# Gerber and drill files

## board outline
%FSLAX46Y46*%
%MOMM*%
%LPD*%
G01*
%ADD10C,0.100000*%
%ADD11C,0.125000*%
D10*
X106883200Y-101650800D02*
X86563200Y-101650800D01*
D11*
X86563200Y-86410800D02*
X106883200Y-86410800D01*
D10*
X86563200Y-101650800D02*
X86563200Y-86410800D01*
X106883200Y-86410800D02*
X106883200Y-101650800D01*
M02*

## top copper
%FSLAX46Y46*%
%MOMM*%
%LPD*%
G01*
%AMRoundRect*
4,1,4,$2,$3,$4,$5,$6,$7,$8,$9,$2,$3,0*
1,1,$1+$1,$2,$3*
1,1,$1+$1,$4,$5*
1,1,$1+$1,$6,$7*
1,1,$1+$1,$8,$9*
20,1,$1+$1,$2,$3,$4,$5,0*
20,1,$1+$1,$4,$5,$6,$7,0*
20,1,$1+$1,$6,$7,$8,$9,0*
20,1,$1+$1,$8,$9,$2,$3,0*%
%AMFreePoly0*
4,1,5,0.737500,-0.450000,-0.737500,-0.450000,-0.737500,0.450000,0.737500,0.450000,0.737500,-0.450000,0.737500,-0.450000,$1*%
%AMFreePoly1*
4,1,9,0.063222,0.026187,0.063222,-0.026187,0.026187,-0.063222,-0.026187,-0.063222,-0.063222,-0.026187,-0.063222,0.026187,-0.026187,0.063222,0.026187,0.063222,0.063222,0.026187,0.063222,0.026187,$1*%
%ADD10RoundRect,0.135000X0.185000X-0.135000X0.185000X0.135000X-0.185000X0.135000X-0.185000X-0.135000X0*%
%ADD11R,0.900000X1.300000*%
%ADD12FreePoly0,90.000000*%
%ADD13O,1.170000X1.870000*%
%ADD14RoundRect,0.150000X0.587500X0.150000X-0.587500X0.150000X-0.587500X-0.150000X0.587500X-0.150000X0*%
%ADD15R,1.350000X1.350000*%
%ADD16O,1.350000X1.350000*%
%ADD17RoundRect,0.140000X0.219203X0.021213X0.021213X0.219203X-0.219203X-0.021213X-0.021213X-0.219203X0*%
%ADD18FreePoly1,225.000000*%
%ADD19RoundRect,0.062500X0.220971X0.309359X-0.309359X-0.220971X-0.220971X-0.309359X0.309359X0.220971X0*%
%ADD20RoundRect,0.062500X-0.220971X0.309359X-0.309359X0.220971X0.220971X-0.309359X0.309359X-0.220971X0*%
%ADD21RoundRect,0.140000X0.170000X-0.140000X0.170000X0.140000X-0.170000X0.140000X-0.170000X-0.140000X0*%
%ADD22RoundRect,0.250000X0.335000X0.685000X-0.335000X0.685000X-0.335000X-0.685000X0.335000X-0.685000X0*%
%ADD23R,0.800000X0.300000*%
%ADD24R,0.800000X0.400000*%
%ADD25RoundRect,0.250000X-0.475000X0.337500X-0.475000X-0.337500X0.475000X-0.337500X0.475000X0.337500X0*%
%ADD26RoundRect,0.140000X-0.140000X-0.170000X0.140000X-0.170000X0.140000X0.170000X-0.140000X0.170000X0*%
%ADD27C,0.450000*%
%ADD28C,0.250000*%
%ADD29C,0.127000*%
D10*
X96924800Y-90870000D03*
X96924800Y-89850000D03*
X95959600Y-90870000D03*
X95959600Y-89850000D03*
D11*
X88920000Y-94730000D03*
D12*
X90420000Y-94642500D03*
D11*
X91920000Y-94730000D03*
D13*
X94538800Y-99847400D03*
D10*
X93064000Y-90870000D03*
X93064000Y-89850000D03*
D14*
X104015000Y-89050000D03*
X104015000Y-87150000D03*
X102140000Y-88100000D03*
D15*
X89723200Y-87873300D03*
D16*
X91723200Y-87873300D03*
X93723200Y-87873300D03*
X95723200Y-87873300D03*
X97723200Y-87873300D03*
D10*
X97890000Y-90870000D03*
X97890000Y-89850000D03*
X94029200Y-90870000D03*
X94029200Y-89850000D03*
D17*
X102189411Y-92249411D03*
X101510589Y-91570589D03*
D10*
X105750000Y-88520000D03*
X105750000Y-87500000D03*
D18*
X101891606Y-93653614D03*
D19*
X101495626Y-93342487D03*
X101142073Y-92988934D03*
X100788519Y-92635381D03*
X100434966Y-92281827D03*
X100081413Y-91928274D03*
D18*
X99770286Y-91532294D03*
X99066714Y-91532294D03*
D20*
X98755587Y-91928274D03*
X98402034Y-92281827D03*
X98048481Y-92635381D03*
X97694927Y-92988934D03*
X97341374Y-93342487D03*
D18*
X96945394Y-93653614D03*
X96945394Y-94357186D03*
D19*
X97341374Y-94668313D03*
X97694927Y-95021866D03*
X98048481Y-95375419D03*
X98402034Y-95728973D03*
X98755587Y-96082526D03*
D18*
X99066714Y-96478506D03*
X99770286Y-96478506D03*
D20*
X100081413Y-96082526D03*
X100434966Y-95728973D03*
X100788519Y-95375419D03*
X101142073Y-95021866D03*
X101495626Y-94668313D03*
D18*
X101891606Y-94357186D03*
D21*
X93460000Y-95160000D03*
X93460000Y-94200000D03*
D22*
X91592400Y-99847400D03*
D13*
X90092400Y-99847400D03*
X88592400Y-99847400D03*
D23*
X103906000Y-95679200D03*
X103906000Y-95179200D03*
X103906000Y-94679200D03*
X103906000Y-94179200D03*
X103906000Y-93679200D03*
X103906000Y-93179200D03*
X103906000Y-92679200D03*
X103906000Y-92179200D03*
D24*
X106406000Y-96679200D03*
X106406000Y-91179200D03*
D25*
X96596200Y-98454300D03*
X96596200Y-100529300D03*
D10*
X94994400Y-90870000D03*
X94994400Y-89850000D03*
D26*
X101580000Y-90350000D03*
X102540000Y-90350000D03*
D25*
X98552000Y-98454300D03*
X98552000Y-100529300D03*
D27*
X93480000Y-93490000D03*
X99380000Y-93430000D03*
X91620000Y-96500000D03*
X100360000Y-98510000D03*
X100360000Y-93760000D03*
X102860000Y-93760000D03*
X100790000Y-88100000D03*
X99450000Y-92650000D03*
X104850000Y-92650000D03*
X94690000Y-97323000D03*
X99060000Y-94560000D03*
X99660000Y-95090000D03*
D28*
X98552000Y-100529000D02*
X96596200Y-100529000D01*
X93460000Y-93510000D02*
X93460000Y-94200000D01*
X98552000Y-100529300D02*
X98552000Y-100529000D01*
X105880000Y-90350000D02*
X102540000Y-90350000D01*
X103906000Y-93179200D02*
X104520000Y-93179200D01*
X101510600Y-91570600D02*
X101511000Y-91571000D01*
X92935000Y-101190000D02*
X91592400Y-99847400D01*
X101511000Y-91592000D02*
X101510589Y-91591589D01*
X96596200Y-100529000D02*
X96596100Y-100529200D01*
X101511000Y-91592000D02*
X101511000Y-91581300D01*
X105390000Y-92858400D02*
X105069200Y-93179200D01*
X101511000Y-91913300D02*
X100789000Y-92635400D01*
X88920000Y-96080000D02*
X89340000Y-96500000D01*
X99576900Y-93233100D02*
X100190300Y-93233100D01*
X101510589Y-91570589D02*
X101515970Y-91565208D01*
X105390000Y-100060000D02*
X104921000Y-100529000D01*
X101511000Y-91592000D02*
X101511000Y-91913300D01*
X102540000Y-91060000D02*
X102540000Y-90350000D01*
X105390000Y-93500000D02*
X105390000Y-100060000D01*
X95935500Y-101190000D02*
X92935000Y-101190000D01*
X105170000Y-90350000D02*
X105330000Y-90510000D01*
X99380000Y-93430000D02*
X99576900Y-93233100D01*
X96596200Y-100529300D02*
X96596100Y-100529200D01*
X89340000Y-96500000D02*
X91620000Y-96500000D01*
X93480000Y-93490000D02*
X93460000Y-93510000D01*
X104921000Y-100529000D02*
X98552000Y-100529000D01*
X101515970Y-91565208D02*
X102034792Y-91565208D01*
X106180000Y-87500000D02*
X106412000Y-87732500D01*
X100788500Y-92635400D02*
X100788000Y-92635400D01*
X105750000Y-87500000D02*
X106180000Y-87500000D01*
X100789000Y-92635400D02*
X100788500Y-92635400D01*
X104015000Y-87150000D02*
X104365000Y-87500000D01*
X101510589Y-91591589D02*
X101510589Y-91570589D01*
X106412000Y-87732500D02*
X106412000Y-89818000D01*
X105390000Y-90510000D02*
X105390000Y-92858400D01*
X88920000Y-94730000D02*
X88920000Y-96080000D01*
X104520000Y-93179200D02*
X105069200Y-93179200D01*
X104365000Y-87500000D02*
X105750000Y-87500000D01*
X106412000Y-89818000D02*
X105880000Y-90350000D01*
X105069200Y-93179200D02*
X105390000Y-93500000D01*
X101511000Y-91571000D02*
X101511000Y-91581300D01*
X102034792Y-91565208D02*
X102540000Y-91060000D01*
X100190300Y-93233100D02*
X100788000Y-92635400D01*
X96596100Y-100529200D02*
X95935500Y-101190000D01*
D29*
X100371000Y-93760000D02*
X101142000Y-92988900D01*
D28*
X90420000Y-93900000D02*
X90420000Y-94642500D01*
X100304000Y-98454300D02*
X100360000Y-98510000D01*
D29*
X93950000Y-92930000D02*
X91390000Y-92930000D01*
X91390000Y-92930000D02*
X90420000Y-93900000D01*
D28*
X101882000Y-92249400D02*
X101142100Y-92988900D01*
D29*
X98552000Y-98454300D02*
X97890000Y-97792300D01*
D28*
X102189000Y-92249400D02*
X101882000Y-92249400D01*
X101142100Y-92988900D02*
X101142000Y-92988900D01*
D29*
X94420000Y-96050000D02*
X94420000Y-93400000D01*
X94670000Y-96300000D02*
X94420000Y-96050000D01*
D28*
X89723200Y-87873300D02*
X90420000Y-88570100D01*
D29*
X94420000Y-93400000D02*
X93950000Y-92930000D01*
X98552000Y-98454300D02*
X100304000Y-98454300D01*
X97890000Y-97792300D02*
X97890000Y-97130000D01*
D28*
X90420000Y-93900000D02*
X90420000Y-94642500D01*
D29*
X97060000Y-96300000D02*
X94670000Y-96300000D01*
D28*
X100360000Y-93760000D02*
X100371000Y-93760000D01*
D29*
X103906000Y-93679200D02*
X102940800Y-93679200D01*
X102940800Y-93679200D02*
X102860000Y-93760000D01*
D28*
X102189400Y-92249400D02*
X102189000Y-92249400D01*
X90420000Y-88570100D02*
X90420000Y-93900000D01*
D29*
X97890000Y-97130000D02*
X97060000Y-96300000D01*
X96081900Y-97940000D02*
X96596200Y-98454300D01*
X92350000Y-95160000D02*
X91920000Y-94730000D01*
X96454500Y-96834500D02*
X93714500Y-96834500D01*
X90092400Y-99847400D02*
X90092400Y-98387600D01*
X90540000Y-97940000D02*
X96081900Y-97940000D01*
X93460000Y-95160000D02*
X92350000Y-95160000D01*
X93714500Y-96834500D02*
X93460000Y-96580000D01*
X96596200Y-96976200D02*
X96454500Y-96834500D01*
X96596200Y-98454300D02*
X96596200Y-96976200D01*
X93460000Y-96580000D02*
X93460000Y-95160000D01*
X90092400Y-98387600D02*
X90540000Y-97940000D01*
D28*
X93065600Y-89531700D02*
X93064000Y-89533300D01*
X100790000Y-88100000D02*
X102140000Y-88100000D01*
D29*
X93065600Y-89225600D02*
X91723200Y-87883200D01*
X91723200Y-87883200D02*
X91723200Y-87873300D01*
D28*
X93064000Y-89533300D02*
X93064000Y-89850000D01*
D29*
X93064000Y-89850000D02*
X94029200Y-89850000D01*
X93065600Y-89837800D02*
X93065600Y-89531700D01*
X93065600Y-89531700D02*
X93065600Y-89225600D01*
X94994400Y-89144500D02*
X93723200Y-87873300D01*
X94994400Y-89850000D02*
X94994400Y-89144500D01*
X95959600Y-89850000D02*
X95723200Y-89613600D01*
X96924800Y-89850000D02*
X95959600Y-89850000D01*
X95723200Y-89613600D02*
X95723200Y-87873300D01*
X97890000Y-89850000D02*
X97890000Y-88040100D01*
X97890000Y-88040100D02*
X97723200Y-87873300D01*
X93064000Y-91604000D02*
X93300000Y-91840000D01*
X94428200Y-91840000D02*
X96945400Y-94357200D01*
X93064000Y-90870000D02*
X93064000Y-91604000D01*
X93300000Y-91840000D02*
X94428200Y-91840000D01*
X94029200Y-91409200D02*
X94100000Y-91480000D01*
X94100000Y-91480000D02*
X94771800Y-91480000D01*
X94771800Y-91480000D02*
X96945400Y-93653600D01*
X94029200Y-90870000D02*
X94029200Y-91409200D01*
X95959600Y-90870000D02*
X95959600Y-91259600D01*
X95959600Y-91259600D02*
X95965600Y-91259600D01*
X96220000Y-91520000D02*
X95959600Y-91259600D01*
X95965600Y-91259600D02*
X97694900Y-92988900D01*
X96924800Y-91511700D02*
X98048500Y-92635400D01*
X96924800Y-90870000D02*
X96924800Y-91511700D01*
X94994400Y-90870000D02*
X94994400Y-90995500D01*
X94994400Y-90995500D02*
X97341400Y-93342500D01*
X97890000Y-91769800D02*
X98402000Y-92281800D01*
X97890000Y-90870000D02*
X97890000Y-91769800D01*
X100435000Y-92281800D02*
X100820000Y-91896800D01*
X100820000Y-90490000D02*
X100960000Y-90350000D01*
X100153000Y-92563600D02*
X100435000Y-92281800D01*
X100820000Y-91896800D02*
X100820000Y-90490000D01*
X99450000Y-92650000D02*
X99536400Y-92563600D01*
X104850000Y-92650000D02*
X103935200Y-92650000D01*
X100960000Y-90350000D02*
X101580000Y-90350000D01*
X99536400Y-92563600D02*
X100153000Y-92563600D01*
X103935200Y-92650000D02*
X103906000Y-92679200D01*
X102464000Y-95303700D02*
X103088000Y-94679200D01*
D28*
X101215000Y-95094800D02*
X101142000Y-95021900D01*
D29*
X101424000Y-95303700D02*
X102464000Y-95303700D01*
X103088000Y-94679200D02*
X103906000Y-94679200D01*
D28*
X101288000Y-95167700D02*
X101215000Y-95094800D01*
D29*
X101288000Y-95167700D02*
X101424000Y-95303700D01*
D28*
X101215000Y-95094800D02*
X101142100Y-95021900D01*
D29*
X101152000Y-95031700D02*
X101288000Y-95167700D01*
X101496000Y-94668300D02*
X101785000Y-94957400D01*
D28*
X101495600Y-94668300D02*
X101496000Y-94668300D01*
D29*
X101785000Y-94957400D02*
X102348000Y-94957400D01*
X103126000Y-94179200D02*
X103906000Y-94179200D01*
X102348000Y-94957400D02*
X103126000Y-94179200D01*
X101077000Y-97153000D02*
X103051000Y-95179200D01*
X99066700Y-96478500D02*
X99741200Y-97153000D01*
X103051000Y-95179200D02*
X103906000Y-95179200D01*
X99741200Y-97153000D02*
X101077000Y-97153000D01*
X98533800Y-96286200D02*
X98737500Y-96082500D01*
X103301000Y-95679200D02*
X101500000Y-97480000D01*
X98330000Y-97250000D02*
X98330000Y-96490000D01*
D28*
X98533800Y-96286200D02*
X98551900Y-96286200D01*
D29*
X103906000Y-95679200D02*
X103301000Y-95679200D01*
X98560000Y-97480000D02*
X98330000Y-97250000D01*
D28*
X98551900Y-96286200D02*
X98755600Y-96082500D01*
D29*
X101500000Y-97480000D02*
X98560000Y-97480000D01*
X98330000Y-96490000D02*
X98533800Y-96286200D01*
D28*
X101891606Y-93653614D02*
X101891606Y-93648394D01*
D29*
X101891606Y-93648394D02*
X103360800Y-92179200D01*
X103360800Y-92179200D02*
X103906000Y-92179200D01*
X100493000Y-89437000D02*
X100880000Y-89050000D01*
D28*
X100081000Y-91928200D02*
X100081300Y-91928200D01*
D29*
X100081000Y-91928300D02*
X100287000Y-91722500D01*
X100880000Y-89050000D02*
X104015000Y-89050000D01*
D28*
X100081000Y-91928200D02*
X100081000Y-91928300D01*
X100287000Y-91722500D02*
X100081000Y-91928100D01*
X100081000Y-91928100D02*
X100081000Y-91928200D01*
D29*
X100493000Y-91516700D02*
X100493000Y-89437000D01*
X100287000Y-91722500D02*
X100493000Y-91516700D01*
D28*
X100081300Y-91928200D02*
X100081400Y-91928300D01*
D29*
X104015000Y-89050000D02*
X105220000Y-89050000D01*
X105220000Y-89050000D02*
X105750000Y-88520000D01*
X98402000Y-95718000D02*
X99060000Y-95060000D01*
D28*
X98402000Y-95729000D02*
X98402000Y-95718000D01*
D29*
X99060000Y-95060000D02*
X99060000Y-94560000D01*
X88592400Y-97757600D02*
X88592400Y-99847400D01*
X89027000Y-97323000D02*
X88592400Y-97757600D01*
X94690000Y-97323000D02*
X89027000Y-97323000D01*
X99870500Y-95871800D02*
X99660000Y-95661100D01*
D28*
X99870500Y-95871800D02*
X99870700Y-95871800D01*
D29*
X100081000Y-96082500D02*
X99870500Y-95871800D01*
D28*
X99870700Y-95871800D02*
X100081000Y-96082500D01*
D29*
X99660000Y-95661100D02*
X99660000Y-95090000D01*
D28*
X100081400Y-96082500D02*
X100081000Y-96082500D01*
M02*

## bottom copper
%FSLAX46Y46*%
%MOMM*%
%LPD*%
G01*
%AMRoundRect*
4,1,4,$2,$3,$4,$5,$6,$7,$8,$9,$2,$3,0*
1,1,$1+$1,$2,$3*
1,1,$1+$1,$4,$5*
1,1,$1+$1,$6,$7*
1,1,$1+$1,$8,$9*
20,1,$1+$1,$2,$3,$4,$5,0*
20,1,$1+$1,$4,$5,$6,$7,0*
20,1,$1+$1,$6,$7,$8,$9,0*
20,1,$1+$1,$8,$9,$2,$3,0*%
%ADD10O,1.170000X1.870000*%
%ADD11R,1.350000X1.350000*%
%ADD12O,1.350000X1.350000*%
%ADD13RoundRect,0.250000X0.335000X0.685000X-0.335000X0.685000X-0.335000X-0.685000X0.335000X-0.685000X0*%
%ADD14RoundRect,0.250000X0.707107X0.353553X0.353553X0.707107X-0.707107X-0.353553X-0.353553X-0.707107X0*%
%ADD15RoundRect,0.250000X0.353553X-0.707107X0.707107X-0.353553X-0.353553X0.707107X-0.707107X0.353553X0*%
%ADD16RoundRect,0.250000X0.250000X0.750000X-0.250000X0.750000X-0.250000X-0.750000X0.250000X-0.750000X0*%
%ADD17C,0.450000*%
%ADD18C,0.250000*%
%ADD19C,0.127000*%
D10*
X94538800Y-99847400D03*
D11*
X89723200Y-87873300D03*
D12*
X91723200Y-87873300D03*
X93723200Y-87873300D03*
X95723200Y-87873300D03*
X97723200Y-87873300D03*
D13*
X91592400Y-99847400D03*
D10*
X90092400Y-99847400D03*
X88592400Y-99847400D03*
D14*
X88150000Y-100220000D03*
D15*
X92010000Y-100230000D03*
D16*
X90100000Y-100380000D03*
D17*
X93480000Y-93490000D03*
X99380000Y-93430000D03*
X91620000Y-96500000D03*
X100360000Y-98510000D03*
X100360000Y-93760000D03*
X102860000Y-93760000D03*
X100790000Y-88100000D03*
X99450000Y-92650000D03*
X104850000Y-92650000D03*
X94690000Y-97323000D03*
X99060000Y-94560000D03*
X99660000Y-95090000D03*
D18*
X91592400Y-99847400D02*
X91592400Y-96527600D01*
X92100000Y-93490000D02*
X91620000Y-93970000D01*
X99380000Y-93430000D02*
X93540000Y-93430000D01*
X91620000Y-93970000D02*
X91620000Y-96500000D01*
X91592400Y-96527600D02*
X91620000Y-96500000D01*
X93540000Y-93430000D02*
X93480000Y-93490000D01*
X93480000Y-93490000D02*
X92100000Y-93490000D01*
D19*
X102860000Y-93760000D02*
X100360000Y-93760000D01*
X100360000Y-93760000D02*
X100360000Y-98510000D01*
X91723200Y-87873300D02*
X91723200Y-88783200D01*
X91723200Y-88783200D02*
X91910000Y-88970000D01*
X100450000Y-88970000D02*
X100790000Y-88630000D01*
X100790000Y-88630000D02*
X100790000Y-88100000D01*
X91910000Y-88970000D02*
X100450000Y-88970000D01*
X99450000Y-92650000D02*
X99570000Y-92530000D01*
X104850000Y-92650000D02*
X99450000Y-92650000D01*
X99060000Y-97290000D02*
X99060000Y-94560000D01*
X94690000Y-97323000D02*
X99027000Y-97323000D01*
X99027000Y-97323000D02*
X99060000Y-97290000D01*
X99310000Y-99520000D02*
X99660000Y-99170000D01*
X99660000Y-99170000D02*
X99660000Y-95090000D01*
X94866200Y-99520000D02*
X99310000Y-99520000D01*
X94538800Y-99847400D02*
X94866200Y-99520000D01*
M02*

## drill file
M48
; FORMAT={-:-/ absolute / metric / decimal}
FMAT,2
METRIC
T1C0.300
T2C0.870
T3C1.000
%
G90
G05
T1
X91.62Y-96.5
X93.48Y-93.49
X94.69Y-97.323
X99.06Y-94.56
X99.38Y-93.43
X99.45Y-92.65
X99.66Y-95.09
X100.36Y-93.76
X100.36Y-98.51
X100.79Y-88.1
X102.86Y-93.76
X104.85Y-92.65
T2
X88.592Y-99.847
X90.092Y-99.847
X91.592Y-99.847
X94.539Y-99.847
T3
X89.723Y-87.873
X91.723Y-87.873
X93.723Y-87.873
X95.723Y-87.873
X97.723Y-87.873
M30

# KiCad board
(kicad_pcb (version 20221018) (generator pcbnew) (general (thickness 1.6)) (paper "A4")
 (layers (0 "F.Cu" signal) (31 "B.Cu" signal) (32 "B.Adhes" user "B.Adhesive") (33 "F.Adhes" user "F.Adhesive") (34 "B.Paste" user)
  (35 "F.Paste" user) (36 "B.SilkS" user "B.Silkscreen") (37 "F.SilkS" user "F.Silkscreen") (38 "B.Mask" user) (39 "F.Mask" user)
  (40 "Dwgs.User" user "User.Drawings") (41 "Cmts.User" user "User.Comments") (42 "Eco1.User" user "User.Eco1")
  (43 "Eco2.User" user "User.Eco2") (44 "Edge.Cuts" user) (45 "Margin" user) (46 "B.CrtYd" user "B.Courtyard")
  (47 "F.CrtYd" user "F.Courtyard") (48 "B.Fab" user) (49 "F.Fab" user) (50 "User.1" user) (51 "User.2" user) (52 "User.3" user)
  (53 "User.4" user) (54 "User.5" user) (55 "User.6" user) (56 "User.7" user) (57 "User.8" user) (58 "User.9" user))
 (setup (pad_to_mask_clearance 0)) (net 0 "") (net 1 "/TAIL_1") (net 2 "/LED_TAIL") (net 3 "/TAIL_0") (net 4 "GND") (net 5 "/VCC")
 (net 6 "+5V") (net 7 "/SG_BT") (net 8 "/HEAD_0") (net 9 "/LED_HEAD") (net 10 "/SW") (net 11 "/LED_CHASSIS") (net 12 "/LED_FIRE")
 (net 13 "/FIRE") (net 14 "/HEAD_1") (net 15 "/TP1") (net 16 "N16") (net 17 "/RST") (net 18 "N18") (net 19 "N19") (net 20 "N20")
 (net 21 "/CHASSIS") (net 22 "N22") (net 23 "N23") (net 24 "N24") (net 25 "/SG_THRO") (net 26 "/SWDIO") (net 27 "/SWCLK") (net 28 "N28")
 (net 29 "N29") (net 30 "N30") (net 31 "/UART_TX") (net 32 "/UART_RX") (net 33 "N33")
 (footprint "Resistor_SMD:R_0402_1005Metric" (layer "F.Cu") (at 96.9248 90.36 90)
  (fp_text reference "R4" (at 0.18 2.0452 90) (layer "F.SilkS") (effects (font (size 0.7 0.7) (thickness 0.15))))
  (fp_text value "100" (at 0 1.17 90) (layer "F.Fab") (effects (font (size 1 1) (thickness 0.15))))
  (pad "1" smd roundrect (at -0.51 0 90) (size 0.54 0.64) (layers "F.Cu" "F.Paste" "F.Mask") (roundrect_rratio 0.25) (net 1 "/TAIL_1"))
  (pad "2" smd roundrect (at 0.51 0 90) (size 0.54 0.64) (layers "F.Cu" "F.Paste" "F.Mask") (roundrect_rratio 0.25) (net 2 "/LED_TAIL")))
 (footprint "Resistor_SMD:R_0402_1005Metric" (layer "F.Cu") (at 95.9596 90.36 90)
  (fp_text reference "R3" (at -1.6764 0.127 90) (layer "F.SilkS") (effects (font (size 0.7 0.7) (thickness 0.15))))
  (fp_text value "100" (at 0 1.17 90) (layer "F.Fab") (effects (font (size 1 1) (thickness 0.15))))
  (pad "1" smd roundrect (at -0.51 0 90) (size 0.54 0.64) (layers "F.Cu" "F.Paste" "F.Mask") (roundrect_rratio 0.25) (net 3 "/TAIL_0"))
  (pad "2" smd roundrect (at 0.51 0 90) (size 0.54 0.64) (layers "F.Cu" "F.Paste" "F.Mask") (roundrect_rratio 0.25) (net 2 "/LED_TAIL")))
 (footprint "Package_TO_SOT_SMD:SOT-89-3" (layer "F.Cu") (at 90.42 92.78 90)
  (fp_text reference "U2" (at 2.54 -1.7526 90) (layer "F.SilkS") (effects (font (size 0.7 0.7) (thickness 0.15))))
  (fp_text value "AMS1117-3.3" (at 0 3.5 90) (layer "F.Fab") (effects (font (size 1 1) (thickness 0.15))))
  (pad "1" smd rect (at -1.95 -1.5 90) (size 1.3 0.9) (layers "F.Cu" "F.Paste" "F.Mask") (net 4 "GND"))
  (pad "2" smd custom (at -1.8625 0 90) (size 1.475 0.9) (layers "F.Cu" "F.Paste" "F.Mask") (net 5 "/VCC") (zone_connect 2)
   (thermal_bridge_angle 45) (options (clearance outline) (anchor rect)) (primitives))
  (pad "3" smd rect (at -1.95 1.5 90) (size 1.3 0.9) (layers "F.Cu" "F.Paste" "F.Mask") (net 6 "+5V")))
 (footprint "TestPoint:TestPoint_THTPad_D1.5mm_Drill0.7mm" (layer "F.Cu") (at 94.5388 99.8474)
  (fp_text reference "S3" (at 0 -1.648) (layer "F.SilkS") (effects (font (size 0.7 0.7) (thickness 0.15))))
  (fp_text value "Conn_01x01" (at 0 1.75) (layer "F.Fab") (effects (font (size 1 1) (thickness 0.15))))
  (pad "1" thru_hole oval (at 0 0) (size 1.17 1.87) (drill 0.87) (layers "*.Cu" "*.Mask") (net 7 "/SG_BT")))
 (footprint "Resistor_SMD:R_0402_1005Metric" (layer "F.Cu") (at 93.064 90.36 90)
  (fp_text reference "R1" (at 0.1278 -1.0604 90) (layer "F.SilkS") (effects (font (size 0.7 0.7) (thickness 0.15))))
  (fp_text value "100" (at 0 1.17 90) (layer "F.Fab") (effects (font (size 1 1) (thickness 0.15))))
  (pad "1" smd roundrect (at -0.51 0 90) (size 0.54 0.64) (layers "F.Cu" "F.Paste" "F.Mask") (roundrect_rratio 0.25) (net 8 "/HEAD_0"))
  (pad "2" smd roundrect (at 0.51 0 90) (size 0.54 0.64) (layers "F.Cu" "F.Paste" "F.Mask") (roundrect_rratio 0.25) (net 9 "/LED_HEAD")))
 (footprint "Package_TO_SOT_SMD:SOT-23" (layer "F.Cu") (at 103.0775 88.1 180)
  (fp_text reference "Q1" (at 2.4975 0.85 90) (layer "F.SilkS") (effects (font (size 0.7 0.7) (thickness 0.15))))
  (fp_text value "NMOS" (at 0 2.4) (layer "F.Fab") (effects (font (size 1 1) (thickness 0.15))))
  (pad "1" smd roundrect (at -0.9375 -0.95 180) (size 1.475 0.6) (layers "F.Cu" "F.Paste" "F.Mask") (roundrect_rratio 0.25) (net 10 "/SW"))
  (pad "2" smd roundrect (at -0.9375 0.95 180) (size 1.475 0.6) (layers "F.Cu" "F.Paste" "F.Mask") (roundrect_rratio 0.25) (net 4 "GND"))
  (pad "3" smd roundrect (at 0.9375 0 180) (size 1.475 0.6) (layers "F.Cu" "F.Paste" "F.Mask") (roundrect_rratio 0.25) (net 9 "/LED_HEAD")))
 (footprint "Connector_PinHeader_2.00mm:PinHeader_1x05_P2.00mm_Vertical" (layer "F.Cu") (at 89.7232 87.8733 90)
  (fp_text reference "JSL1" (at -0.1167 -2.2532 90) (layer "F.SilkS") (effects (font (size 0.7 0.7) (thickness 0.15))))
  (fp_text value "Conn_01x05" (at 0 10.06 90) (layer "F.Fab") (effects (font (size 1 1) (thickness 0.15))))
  (pad "1" thru_hole rect (at 0 0 90) (size 1.35 1.35) (drill 1) (layers "*.Cu" "*.Mask") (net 5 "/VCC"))
  (pad "2" thru_hole oval (at 0 2 90) (size 1.35 1.35) (drill 1) (layers "*.Cu" "*.Mask") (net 9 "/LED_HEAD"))
  (pad "3" thru_hole oval (at 0 4 90) (size 1.35 1.35) (drill 1) (layers "*.Cu" "*.Mask") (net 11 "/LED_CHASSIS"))
  (pad "4" thru_hole oval (at 0 6 90) (size 1.35 1.35) (drill 1) (layers "*.Cu" "*.Mask") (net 2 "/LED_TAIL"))
  (pad "5" thru_hole oval (at 0 8 90) (size 1.35 1.35) (drill 1) (layers "*.Cu" "*.Mask") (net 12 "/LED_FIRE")))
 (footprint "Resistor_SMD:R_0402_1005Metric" (layer "F.Cu") (at 97.89 90.36 90)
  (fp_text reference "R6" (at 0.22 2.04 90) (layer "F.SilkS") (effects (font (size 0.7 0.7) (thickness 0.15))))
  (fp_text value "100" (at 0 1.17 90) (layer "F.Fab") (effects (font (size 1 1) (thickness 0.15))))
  (pad "1" smd roundrect (at -0.51 0 90) (size 0.54 0.64) (layers "F.Cu" "F.Paste" "F.Mask") (roundrect_rratio 0.25) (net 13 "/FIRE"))
  (pad "2" smd roundrect (at 0.51 0 90) (size 0.54 0.64) (layers "F.Cu" "F.Paste" "F.Mask") (roundrect_rratio 0.25) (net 12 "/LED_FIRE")))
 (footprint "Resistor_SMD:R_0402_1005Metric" (layer "F.Cu") (at 94.0292 90.36 90)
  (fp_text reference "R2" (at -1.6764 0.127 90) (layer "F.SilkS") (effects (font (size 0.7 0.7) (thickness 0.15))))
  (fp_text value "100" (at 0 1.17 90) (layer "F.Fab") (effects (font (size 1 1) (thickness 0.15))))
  (pad "1" smd roundrect (at -0.51 0 90) (size 0.54 0.64) (layers "F.Cu" "F.Paste" "F.Mask") (roundrect_rratio 0.25) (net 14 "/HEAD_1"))
  (pad "2" smd roundrect (at 0.51 0 90) (size 0.54 0.64) (layers "F.Cu" "F.Paste" "F.Mask") (roundrect_rratio 0.25) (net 9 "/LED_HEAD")))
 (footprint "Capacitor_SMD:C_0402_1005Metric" (layer "F.Cu") (at 101.85 91.91 135)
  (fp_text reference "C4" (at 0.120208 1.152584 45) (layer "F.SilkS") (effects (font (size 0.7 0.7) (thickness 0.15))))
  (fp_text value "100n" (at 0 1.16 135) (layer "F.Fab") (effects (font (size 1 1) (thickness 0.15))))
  (pad "1" smd roundrect (at -0.48 0 135) (size 0.56 0.62) (layers "F.Cu" "F.Paste" "F.Mask") (roundrect_rratio 0.25) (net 5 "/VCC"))
  (pad "2" smd roundrect (at 0.48 0 135) (size 0.56 0.62) (layers "F.Cu" "F.Paste" "F.Mask") (roundrect_rratio 0.25) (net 4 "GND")))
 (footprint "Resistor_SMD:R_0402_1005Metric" (layer "F.Cu") (at 105.75 88.01 90)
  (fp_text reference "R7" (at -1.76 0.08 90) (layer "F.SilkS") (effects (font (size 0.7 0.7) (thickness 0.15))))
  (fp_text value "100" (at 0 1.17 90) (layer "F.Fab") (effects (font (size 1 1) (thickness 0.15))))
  (pad "1" smd roundrect (at -0.51 0 90) (size 0.54 0.64) (layers "F.Cu" "F.Paste" "F.Mask") (roundrect_rratio 0.25) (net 10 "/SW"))
  (pad "2" smd roundrect (at 0.51 0 90) (size 0.54 0.64) (layers "F.Cu" "F.Paste" "F.Mask") (roundrect_rratio 0.25) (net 4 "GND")))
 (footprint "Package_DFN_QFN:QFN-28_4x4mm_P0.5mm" (layer "F.Cu") (at 99.4185 94.0054 -135)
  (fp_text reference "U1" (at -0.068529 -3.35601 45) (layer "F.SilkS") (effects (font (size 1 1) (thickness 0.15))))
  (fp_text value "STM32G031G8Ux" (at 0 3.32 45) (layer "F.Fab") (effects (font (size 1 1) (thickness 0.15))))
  (pad "1" smd custom (at -1.9975 -1.5 225) (size 0.136863 0.136863) (layers "F.Cu" "F.Paste" "F.Mask") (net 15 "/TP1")
   (thermal_bridge_angle 45) (options (clearance outline) (anchor circle)) (primitives))
  (pad "2" smd roundrect (at -1.9375 -1 225) (size 0.875 0.25) (layers "F.Cu" "F.Paste" "F.Mask") (roundrect_rratio 0.25) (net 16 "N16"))
  (pad "3" smd roundrect (at -1.9375 -0.5 225) (size 0.875 0.25) (layers "F.Cu" "F.Paste" "F.Mask") (roundrect_rratio 0.25) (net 5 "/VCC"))
  (pad "4" smd roundrect (at -1.9375 0 225) (size 0.875 0.25) (layers "F.Cu" "F.Paste" "F.Mask") (roundrect_rratio 0.25) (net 4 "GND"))
  (pad "5" smd roundrect (at -1.9375 0.5 225) (size 0.875 0.25) (layers "F.Cu" "F.Paste" "F.Mask") (roundrect_rratio 0.25) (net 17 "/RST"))
  (pad "6" smd roundrect (at -1.9375 1 225) (size 0.875 0.25) (layers "F.Cu" "F.Paste" "F.Mask") (roundrect_rratio 0.25) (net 10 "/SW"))
  (pad "7" smd custom (at -1.9975 1.5 225) (size 0.136863 0.136863) (layers "F.Cu" "F.Paste" "F.Mask") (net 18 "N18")
   (thermal_bridge_angle 45) (options (clearance outline) (anchor circle)) (primitives))
  (pad "8" smd custom (at -1.5 1.9975 225) (size 0.136863 0.136863) (layers "F.Cu" "F.Paste" "F.Mask") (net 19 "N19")
   (thermal_bridge_angle 45) (options (clearance outline) (anchor circle)) (primitives))
  (pad "9" smd roundrect (at -1 1.9375 225) (size 0.25 0.875) (layers "F.Cu" "F.Paste" "F.Mask") (roundrect_rratio 0.25) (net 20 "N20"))
  (pad "10" smd roundrect (at -0.5 1.9375 225) (size 0.25 0.875) (layers "F.Cu" "F.Paste" "F.Mask") (roundrect_rratio 0.25) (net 13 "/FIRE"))
  (pad "11" smd roundrect (at 0 1.9375 225) (size 0.25 0.875) (layers "F.Cu" "F.Paste" "F.Mask") (roundrect_rratio 0.25) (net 1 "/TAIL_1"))
  (pad "12" smd roundrect (at 0.5 1.9375 225) (size 0.25 0.875) (layers "F.Cu" "F.Paste" "F.Mask") (roundrect_rratio 0.25) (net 3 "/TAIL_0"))
  (pad "13" smd roundrect (at 1 1.9375 225) (size 0.25 0.875) (layers "F.Cu" "F.Paste" "F.Mask") (roundrect_rratio 0.25) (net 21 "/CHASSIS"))
  (pad "14" smd custom (at 1.5 1.9975 225) (size 0.136863 0.136863) (layers "F.Cu" "F.Paste" "F.Mask") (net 14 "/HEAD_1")
   (thermal_bridge_angle 45) (options (clearance outline) (anchor circle)) (primitives))
  (pad "15" smd custom (at 1.9975 1.5 225) (size 0.136863 0.136863) (layers "F.Cu" "F.Paste" "F.Mask") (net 8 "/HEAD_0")
   (thermal_bridge_angle 45) (options (clearance outline) (anchor circle)) (primitives))
  (pad "16" smd roundrect (at 1.9375 1 225) (size 0.875 0.25) (layers "F.Cu" "F.Paste" "F.Mask") (roundrect_rratio 0.25) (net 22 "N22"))
  (pad "17" smd roundrect (at 1.9375 0.5 225) (size 0.875 0.25) (layers "F.Cu" "F.Paste" "F.Mask") (roundrect_rratio 0.25) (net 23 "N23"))
  (pad "18" smd roundrect (at 1.9375 0 225) (size 0.875 0.25) (layers "F.Cu" "F.Paste" "F.Mask") (roundrect_rratio 0.25) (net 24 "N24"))
  (pad "19" smd roundrect (at 1.9375 -0.5 225) (size 0.875 0.25) (layers "F.Cu" "F.Paste" "F.Mask") (roundrect_rratio 0.25)
   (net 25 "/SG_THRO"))
  (pad "20" smd roundrect (at 1.9375 -1 225) (size 0.875 0.25) (layers "F.Cu" "F.Paste" "F.Mask") (roundrect_rratio 0.25) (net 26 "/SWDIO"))
  (pad "21" smd custom (at 1.9975 -1.5 225) (size 0.136863 0.136863) (layers "F.Cu" "F.Paste" "F.Mask") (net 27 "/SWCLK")
   (thermal_bridge_angle 45) (options (clearance outline) (anchor circle)) (primitives))
  (pad "22" smd custom (at 1.5 -1.9975 225) (size 0.136863 0.136863) (layers "F.Cu" "F.Paste" "F.Mask") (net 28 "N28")
   (thermal_bridge_angle 45) (options (clearance outline) (anchor circle)) (primitives))
  (pad "23" smd roundrect (at 1 -1.9375 225) (size 0.25 0.875) (layers "F.Cu" "F.Paste" "F.Mask") (roundrect_rratio 0.25) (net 7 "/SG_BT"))
  (pad "24" smd roundrect (at 0.5 -1.9375 225) (size 0.25 0.875) (layers "F.Cu" "F.Paste" "F.Mask") (roundrect_rratio 0.25) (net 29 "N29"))
  (pad "25" smd roundrect (at 0 -1.9375 225) (size 0.25 0.875) (layers "F.Cu" "F.Paste" "F.Mask") (roundrect_rratio 0.25) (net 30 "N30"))
  (pad "26" smd roundrect (at -0.5 -1.9375 225) (size 0.25 0.875) (layers "F.Cu" "F.Paste" "F.Mask") (roundrect_rratio 0.25)
   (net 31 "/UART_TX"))
  (pad "27" smd roundrect (at -1 -1.9375 225) (size 0.25 0.875) (layers "F.Cu" "F.Paste" "F.Mask") (roundrect_rratio 0.25)
   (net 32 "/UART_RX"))
  (pad "28" smd custom (at -1.5 -1.9975 225) (size 0.136863 0.136863) (layers "F.Cu" "F.Paste" "F.Mask") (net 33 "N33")
   (thermal_bridge_angle 45) (options (clearance outline) (anchor circle)) (primitives)))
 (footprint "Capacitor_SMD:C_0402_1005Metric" (layer "F.Cu") (at 93.46 94.68 90)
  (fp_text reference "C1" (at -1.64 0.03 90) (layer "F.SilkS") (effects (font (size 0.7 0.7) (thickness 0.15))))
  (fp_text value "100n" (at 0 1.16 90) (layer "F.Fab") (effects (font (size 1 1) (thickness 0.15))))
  (pad "1" smd roundrect (at -0.48 0 90) (size 0.56 0.62) (layers "F.Cu" "F.Paste" "F.Mask") (roundrect_rratio 0.25) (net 6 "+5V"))
  (pad "2" smd roundrect (at 0.48 0 90) (size 0.56 0.62) (layers "F.Cu" "F.Paste" "F.Mask") (roundrect_rratio 0.25) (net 4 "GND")))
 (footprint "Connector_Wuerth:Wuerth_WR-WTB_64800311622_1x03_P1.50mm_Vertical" (layer "F.Cu") (at 91.5924 99.8474 180)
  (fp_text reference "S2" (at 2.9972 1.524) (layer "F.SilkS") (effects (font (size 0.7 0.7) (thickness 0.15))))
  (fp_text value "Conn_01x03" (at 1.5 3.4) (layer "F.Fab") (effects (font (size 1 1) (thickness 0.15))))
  (pad "1" thru_hole roundrect (at 0 0 180) (size 1.17 1.87) (drill 0.87) (layers "*.Cu" "*.Mask") (roundrect_rratio 0.213675) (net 4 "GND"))
  (pad "2" thru_hole oval (at 1.5 0 180) (size 1.17 1.87) (drill 0.87) (layers "*.Cu" "*.Mask") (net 6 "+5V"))
  (pad "3" thru_hole oval (at 3 0 180) (size 1.17 1.87) (drill 0.87) (layers "*.Cu" "*.Mask") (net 25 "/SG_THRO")))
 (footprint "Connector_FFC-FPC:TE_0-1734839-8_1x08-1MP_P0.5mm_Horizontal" (layer "F.Cu") (at 104.831 93.9292 90)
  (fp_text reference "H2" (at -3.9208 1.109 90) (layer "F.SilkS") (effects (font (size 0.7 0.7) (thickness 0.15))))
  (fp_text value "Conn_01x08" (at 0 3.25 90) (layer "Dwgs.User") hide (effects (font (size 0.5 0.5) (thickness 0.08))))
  (pad "1" smd rect (at -1.75 -0.925 90) (size 0.3 0.8) (layers "F.Cu" "F.Paste" "F.Mask") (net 26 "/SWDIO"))
  (pad "2" smd rect (at -1.25 -0.925 90) (size 0.3 0.8) (layers "F.Cu" "F.Paste" "F.Mask") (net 27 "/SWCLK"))
  (pad "3" smd rect (at -0.75 -0.925 90) (size 0.3 0.8) (layers "F.Cu" "F.Paste" "F.Mask") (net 31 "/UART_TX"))
  (pad "4" smd rect (at -0.25 -0.925 90) (size 0.3 0.8) (layers "F.Cu" "F.Paste" "F.Mask") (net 32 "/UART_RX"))
  (pad "5" smd rect (at 0.25 -0.925 90) (size 0.3 0.8) (layers "F.Cu" "F.Paste" "F.Mask") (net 5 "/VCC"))
  (pad "6" smd rect (at 0.75 -0.925 90) (size 0.3 0.8) (layers "F.Cu" "F.Paste" "F.Mask") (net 4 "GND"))
  (pad "7" smd rect (at 1.25 -0.925 90) (size 0.3 0.8) (layers "F.Cu" "F.Paste" "F.Mask") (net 17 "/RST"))
  (pad "8" smd rect (at 1.75 -0.925 90) (size 0.3 0.8) (layers "F.Cu" "F.Paste" "F.Mask") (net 15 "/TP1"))
  (pad "MP" smd rect (at -2.75 1.575 90) (size 0.4 0.8) (layers "F.Cu" "F.Paste" "F.Mask"))
  (pad "MP" smd rect (at 2.75 1.575 90) (size 0.4 0.8) (layers "F.Cu" "F.Paste" "F.Mask")))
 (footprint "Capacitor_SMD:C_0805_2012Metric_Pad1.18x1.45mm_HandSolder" (layer "F.Cu") (at 96.5962 99.4918 -90)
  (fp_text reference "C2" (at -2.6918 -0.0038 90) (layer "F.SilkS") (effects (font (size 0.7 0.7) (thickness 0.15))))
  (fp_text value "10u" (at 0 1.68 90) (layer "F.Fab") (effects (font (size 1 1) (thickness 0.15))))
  (pad "1" smd roundrect (at -1.0375 0 270) (size 1.175 1.45) (layers "F.Cu" "F.Paste" "F.Mask") (roundrect_rratio 0.212766) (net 6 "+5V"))
  (pad "2" smd roundrect (at 1.0375 0 270) (size 1.175 1.45) (layers "F.Cu" "F.Paste" "F.Mask") (roundrect_rratio 0.212766) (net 4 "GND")))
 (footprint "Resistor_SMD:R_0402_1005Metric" (layer "F.Cu") (at 94.9944 90.36 90)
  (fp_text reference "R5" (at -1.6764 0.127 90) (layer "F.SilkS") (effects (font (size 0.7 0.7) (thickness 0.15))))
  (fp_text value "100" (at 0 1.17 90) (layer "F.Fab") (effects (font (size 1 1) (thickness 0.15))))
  (pad "1" smd roundrect (at -0.51 0 90) (size 0.54 0.64) (layers "F.Cu" "F.Paste" "F.Mask") (roundrect_rratio 0.25) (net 21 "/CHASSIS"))
  (pad "2" smd roundrect (at 0.51 0 90) (size 0.54 0.64) (layers "F.Cu" "F.Paste" "F.Mask") (roundrect_rratio 0.25) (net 11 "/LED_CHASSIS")))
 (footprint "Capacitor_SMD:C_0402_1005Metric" (layer "F.Cu") (at 102.06 90.35)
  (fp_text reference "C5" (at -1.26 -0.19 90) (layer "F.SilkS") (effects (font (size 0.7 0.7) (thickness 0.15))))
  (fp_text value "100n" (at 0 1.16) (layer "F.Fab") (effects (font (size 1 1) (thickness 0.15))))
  (pad "1" smd roundrect (at -0.48 0) (size 0.56 0.62) (layers "F.Cu" "F.Paste" "F.Mask") (roundrect_rratio 0.25) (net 17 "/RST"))
  (pad "2" smd roundrect (at 0.48 0) (size 0.56 0.62) (layers "F.Cu" "F.Paste" "F.Mask") (roundrect_rratio 0.25) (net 4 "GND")))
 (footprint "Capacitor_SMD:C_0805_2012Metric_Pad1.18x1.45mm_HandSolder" (layer "F.Cu") (at 98.552 99.4918 -90)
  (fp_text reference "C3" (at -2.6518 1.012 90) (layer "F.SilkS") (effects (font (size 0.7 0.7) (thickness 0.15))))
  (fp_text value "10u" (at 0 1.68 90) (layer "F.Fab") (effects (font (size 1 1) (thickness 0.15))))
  (pad "1" smd roundrect (at -1.0375 0 270) (size 1.175 1.45) (layers "F.Cu" "F.Paste" "F.Mask") (roundrect_rratio 0.212766) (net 5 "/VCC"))
  (pad "2" smd roundrect (at 1.0375 0 270) (size 1.175 1.45) (layers "F.Cu" "F.Paste" "F.Mask") (roundrect_rratio 0.212766) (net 4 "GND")))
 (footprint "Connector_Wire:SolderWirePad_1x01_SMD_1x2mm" (layer "B.Cu") (at 88.15 100.22 135)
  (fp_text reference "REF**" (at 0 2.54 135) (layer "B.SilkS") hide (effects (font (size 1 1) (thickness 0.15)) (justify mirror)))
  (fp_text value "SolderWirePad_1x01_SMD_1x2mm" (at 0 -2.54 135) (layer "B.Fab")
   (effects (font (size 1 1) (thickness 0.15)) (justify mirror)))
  (pad "1" smd roundrect (at 0 0 135) (size 1 2) (layers "B.Cu" "B.Paste" "B.Mask") (roundrect_rratio 0.25) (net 25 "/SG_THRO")))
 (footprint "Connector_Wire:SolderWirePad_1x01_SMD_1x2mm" (layer "B.Cu") (at 92.01 100.23 45)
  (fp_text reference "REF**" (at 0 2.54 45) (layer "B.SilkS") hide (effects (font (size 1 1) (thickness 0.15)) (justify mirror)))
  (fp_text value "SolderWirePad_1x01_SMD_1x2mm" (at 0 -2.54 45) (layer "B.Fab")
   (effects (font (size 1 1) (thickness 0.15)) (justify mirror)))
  (pad "1" smd roundrect (at 0 0 45) (size 1 2) (layers "B.Cu" "B.Paste" "B.Mask") (roundrect_rratio 0.25) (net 4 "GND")))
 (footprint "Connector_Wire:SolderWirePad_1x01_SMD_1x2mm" (layer "B.Cu") (at 90.1 100.38 180)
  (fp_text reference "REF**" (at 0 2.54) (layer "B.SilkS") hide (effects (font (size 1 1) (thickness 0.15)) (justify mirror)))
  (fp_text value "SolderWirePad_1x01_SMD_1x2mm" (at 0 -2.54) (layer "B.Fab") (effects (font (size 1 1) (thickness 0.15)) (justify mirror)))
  (pad "1" smd roundrect (at 0 0 180) (size 1 2) (layers "B.Cu" "B.Paste" "B.Mask") (roundrect_rratio 0.25) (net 6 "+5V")))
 (gr_line (start 106.8832 101.6508) (end 86.5632 101.6508) (stroke (width 0.1) (type default)) (layer "Edge.Cuts"))
 (gr_line (start 86.5632 86.4108) (end 106.8832 86.4108) (stroke (width 0.125) (type default)) (layer "Edge.Cuts"))
 (gr_line (start 86.5632 101.6508) (end 86.5632 86.4108) (stroke (width 0.1) (type default)) (layer "Edge.Cuts"))
 (gr_line (start 106.8832 86.4108) (end 106.8832 101.6508) (stroke (width 0.1) (type default)) (layer "Edge.Cuts"))
 (segment (start 98.552 100.529) (end 96.5962 100.529) (width 0.25) (layer "F.Cu") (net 4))
 (segment (start 93.46 93.51) (end 93.46 94.2) (width 0.25) (layer "F.Cu") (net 4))
 (segment (start 98.552 100.5293) (end 98.552 100.529) (width 0.25) (layer "F.Cu") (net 4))
 (segment (start 105.88 90.35) (end 102.54 90.35) (width 0.25) (layer "F.Cu") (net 4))
 (segment (start 103.906 93.1792) (end 104.52 93.1792) (width 0.25) (layer "F.Cu") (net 4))
 (segment (start 101.5106 91.5706) (end 101.511 91.571) (width 0.25) (layer "F.Cu") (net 4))
 (segment (start 92.935 101.19) (end 91.5924 99.8474) (width 0.25) (layer "F.Cu") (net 4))
 (segment (start 101.511 91.592) (end 101.510589 91.591589) (width 0.25) (layer "F.Cu") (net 4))
 (segment (start 96.5962 100.529) (end 96.5961 100.5292) (width 0.25) (layer "F.Cu") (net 4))
 (segment (start 101.511 91.592) (end 101.511 91.5813) (width 0.25) (layer "F.Cu") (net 4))
 (segment (start 105.39 92.8584) (end 105.0692 93.1792) (width 0.25) (layer "F.Cu") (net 4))
 (segment (start 101.511 91.9133) (end 100.789 92.6354) (width 0.25) (layer "F.Cu") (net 4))
 (segment (start 88.92 96.08) (end 89.34 96.5) (width 0.25) (layer "F.Cu") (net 4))
 (segment (start 99.5769 93.2331) (end 100.1903 93.2331) (width 0.25) (layer "F.Cu") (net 4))
 (segment (start 101.510589 91.570589) (end 101.51597 91.565208) (width 0.25) (layer "F.Cu") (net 4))
 (segment (start 105.39 100.06) (end 104.921 100.529) (width 0.25) (layer "F.Cu") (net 4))
 (segment (start 101.511 91.592) (end 101.511 91.9133) (width 0.25) (layer "F.Cu") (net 4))
 (segment (start 102.54 91.06) (end 102.54 90.35) (width 0.25) (layer "F.Cu") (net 4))
 (segment (start 105.39 93.5) (end 105.39 100.06) (width 0.25) (layer "F.Cu") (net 4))
 (segment (start 95.9355 101.19) (end 92.935 101.19) (width 0.25) (layer "F.Cu") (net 4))
 (segment (start 105.17 90.35) (end 105.33 90.51) (width 0.25) (layer "F.Cu") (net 4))
 (segment (start 99.38 93.43) (end 99.5769 93.2331) (width 0.25) (layer "F.Cu") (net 4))
 (segment (start 96.5962 100.5293) (end 96.5961 100.5292) (width 0.25) (layer "F.Cu") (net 4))
 (segment (start 89.34 96.5) (end 91.62 96.5) (width 0.25) (layer "F.Cu") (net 4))
 (segment (start 93.48 93.49) (end 93.46 93.51) (width 0.25) (layer "F.Cu") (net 4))
 (segment (start 104.921 100.529) (end 98.552 100.529) (width 0.25) (layer "F.Cu") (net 4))
 (segment (start 101.51597 91.565208) (end 102.034792 91.565208) (width 0.25) (layer "F.Cu") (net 4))
 (segment (start 106.18 87.5) (end 106.412 87.7325) (width 0.25) (layer "F.Cu") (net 4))
 (segment (start 100.7885 92.6354) (end 100.788 92.6354) (width 0.25) (layer "F.Cu") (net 4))
 (segment (start 105.75 87.5) (end 106.18 87.5) (width 0.25) (layer "F.Cu") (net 4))
 (segment (start 100.789 92.6354) (end 100.7885 92.6354) (width 0.25) (layer "F.Cu") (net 4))
 (segment (start 104.015 87.15) (end 104.365 87.5) (width 0.25) (layer "F.Cu") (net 4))
 (segment (start 101.510589 91.591589) (end 101.510589 91.570589) (width 0.25) (layer "F.Cu") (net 4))
 (segment (start 106.412 87.7325) (end 106.412 89.818) (width 0.25) (layer "F.Cu") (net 4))
 (segment (start 105.39 90.51) (end 105.39 92.8584) (width 0.25) (layer "F.Cu") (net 4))
 (segment (start 88.92 94.73) (end 88.92 96.08) (width 0.25) (layer "F.Cu") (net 4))
 (segment (start 104.52 93.1792) (end 105.0692 93.1792) (width 0.25) (layer "F.Cu") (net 4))
 (segment (start 104.365 87.5) (end 105.75 87.5) (width 0.25) (layer "F.Cu") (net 4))
 (segment (start 106.412 89.818) (end 105.88 90.35) (width 0.25) (layer "F.Cu") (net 4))
 (segment (start 105.0692 93.1792) (end 105.39 93.5) (width 0.25) (layer "F.Cu") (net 4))
 (segment (start 101.511 91.571) (end 101.511 91.5813) (width 0.25) (layer "F.Cu") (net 4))
 (segment (start 102.034792 91.565208) (end 102.54 91.06) (width 0.25) (layer "F.Cu") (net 4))
 (segment (start 100.1903 93.2331) (end 100.788 92.6354) (width 0.25) (layer "F.Cu") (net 4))
 (segment (start 96.5961 100.5292) (end 95.9355 101.19) (width 0.25) (layer "F.Cu") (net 4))
 (via (at 93.48 93.49) (size 0.45) (drill 0.3) (layers "F.Cu" "B.Cu") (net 4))
 (via (at 99.38 93.43) (size 0.45) (drill 0.3) (layers "F.Cu" "B.Cu") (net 4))
 (via (at 91.62 96.5) (size 0.45) (drill 0.3) (layers "F.Cu" "B.Cu") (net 4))
 (segment (start 91.5924 99.8474) (end 91.5924 96.5276) (width 0.25) (layer "B.Cu") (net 4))
 (segment (start 92.1 93.49) (end 91.62 93.97) (width 0.25) (layer "B.Cu") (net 4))
 (segment (start 99.38 93.43) (end 93.54 93.43) (width 0.25) (layer "B.Cu") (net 4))
 (segment (start 91.62 93.97) (end 91.62 96.5) (width 0.25) (layer "B.Cu") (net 4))
 (segment (start 91.5924 96.5276) (end 91.62 96.5) (width 0.25) (layer "B.Cu") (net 4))
 (segment (start 93.54 93.43) (end 93.48 93.49) (width 0.25) (layer "B.Cu") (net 4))
 (segment (start 93.48 93.49) (end 92.1 93.49) (width 0.25) (layer "B.Cu") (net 4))
 (segment (start 100.371 93.76) (end 101.142 92.9889) (width 0.127) (layer "F.Cu") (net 5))
 (segment (start 90.42 93.9) (end 90.42 94.6425) (width 0.25) (layer "F.Cu") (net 5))
 (segment (start 100.304 98.4543) (end 100.36 98.51) (width 0.25) (layer "F.Cu") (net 5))
 (segment (start 93.95 92.93) (end 91.39 92.93) (width 0.127) (layer "F.Cu") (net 5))
 (segment (start 91.39 92.93) (end 90.42 93.9) (width 0.127) (layer "F.Cu") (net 5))
 (segment (start 101.882 92.2494) (end 101.1421 92.9889) (width 0.25) (layer "F.Cu") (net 5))
 (segment (start 98.552 98.4543) (end 97.89 97.7923) (width 0.127) (layer "F.Cu") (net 5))
 (segment (start 102.189 92.2494) (end 101.882 92.2494) (width 0.25) (layer "F.Cu") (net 5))
 (segment (start 101.1421 92.9889) (end 101.142 92.9889) (width 0.25) (layer "F.Cu") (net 5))
 (segment (start 94.42 96.05) (end 94.42 93.4) (width 0.127) (layer "F.Cu") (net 5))
 (segment (start 94.67 96.3) (end 94.42 96.05) (width 0.127) (layer "F.Cu") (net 5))
 (segment (start 89.7232 87.8733) (end 90.42 88.5701) (width 0.25) (layer "F.Cu") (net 5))
 (segment (start 94.42 93.4) (end 93.95 92.93) (width 0.127) (layer "F.Cu") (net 5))
 (segment (start 98.552 98.4543) (end 100.304 98.4543) (width 0.127) (layer "F.Cu") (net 5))
 (segment (start 97.89 97.7923) (end 97.89 97.13) (width 0.127) (layer "F.Cu") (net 5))
 (segment (start 90.42 93.9) (end 90.42 94.6425) (width 0.25) (layer "F.Cu") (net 5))
 (segment (start 97.06 96.3) (end 94.67 96.3) (width 0.127) (layer "F.Cu") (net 5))
 (segment (start 100.36 93.76) (end 100.371 93.76) (width 0.25) (layer "F.Cu") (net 5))
 (segment (start 103.906 93.6792) (end 102.9408 93.6792) (width 0.127) (layer "F.Cu") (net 5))
 (segment (start 102.9408 93.6792) (end 102.86 93.76) (width 0.127) (layer "F.Cu") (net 5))
 (segment (start 102.1894 92.2494) (end 102.189 92.2494) (width 0.25) (layer "F.Cu") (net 5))
 (segment (start 90.42 88.5701) (end 90.42 93.9) (width 0.25) (layer "F.Cu") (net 5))
 (segment (start 97.89 97.13) (end 97.06 96.3) (width 0.127) (layer "F.Cu") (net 5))
 (via (at 100.36 98.51) (size 0.45) (drill 0.3) (layers "F.Cu" "B.Cu") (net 5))
 (via (at 100.36 93.76) (size 0.45) (drill 0.3) (layers "F.Cu" "B.Cu") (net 5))
 (via (at 102.86 93.76) (size 0.45) (drill 0.3) (layers "F.Cu" "B.Cu") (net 5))
 (segment (start 102.86 93.76) (end 100.36 93.76) (width 0.127) (layer "B.Cu") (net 5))
 (segment (start 100.36 93.76) (end 100.36 98.51) (width 0.127) (layer "B.Cu") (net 5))
 (segment (start 96.0819 97.94) (end 96.5962 98.4543) (width 0.127) (layer "F.Cu") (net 6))
 (segment (start 92.35 95.16) (end 91.92 94.73) (width 0.127) (layer "F.Cu") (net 6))
 (segment (start 96.4545 96.8345) (end 93.7145 96.8345) (width 0.127) (layer "F.Cu") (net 6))
 (segment (start 90.0924 99.8474) (end 90.0924 98.3876) (width 0.127) (layer "F.Cu") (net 6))
 (segment (start 90.54 97.94) (end 96.0819 97.94) (width 0.127) (layer "F.Cu") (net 6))
 (segment (start 93.46 95.16) (end 92.35 95.16) (width 0.127) (layer "F.Cu") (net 6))
 (segment (start 93.7145 96.8345) (end 93.46 96.58) (width 0.127) (layer "F.Cu") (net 6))
 (segment (start 96.5962 96.9762) (end 96.4545 96.8345) (width 0.127) (layer "F.Cu") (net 6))
 (segment (start 96.5962 98.4543) (end 96.5962 96.9762) (width 0.127) (layer "F.Cu") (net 6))
 (segment (start 93.46 96.58) (end 93.46 95.16) (width 0.127) (layer "F.Cu") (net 6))
 (segment (start 90.0924 98.3876) (end 90.54 97.94) (width 0.127) (layer "F.Cu") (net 6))
 (segment (start 93.0656 89.5317) (end 93.064 89.5333) (width 0.25) (layer "F.Cu") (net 9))
 (segment (start 100.79 88.1) (end 102.14 88.1) (width 0.25) (layer "F.Cu") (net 9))
 (segment (start 93.0656 89.2256) (end 91.7232 87.8832) (width 0.127) (layer "F.Cu") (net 9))
 (segment (start 91.7232 87.8832) (end 91.7232 87.8733) (width 0.127) (layer "F.Cu") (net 9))
 (segment (start 93.064 89.5333) (end 93.064 89.85) (width 0.25) (layer "F.Cu") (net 9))
 (segment (start 93.064 89.85) (end 94.0292 89.85) (width 0.127) (layer "F.Cu") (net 9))
 (segment (start 93.0656 89.8378) (end 93.0656 89.5317) (width 0.127) (layer "F.Cu") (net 9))
 (segment (start 93.0656 89.5317) (end 93.0656 89.2256) (width 0.127) (layer "F.Cu") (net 9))
 (via (at 100.79 88.1) (size 0.45) (drill 0.3) (layers "F.Cu" "B.Cu") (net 9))
 (segment (start 91.7232 87.8733) (end 91.7232 88.7832) (width 0.127) (layer "B.Cu") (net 9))
 (segment (start 91.7232 88.7832) (end 91.91 88.97) (width 0.127) (layer "B.Cu") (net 9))
 (segment (start 100.45 88.97) (end 100.79 88.63) (width 0.127) (layer "B.Cu") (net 9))
 (segment (start 100.79 88.63) (end 100.79 88.1) (width 0.127) (layer "B.Cu") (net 9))
 (segment (start 91.91 88.97) (end 100.45 88.97) (width 0.127) (layer "B.Cu") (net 9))
 (segment (start 94.9944 89.1445) (end 93.7232 87.8733) (width 0.127) (layer "F.Cu") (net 11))
 (segment (start 94.9944 89.85) (end 94.9944 89.1445) (width 0.127) (layer "F.Cu") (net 11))
 (segment (start 95.9596 89.85) (end 95.7232 89.6136) (width 0.127) (layer "F.Cu") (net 2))
 (segment (start 96.9248 89.85) (end 95.9596 89.85) (width 0.127) (layer "F.Cu") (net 2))
 (segment (start 95.7232 89.6136) (end 95.7232 87.8733) (width 0.127) (layer "F.Cu") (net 2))
 (segment (start 97.89 89.85) (end 97.89 88.0401) (width 0.127) (layer "F.Cu") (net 12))
 (segment (start 97.89 88.0401) (end 97.7232 87.8733) (width 0.127) (layer "F.Cu") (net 12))
 (segment (start 93.064 91.604) (end 93.3 91.84) (width 0.127) (layer "F.Cu") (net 8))
 (segment (start 94.4282 91.84) (end 96.9454 94.3572) (width 0.127) (layer "F.Cu") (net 8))
 (segment (start 93.064 90.87) (end 93.064 91.604) (width 0.127) (layer "F.Cu") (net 8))
 (segment (start 93.3 91.84) (end 94.4282 91.84) (width 0.127) (layer "F.Cu") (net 8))
 (segment (start 94.0292 91.4092) (end 94.1 91.48) (width 0.127) (layer "F.Cu") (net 14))
 (segment (start 94.1 91.48) (end 94.7718 91.48) (width 0.127) (layer "F.Cu") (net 14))
 (segment (start 94.7718 91.48) (end 96.9454 93.6536) (width 0.127) (layer "F.Cu") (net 14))
 (segment (start 94.0292 90.87) (end 94.0292 91.4092) (width 0.127) (layer "F.Cu") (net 14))
 (segment (start 95.9596 90.87) (end 95.9596 91.2596) (width 0.127) (layer "F.Cu") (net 3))
 (segment (start 95.9596 91.2596) (end 95.9656 91.2596) (width 0.127) (layer "F.Cu") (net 3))
 (segment (start 96.22 91.52) (end 95.9596 91.2596) (width 0.127) (layer "F.Cu") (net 3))
 (segment (start 95.9656 91.2596) (end 97.6949 92.9889) (width 0.127) (layer "F.Cu") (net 3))
 (segment (start 96.9248 91.5117) (end 98.0485 92.6354) (width 0.127) (layer "F.Cu") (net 1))
 (segment (start 96.9248 90.87) (end 96.9248 91.5117) (width 0.127) (layer "F.Cu") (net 1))
 (segment (start 94.9944 90.87) (end 94.9944 90.9955) (width 0.127) (layer "F.Cu") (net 21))
 (segment (start 94.9944 90.9955) (end 97.3414 93.3425) (width 0.127) (layer "F.Cu") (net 21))
 (segment (start 97.89 91.7698) (end 98.402 92.2818) (width 0.127) (layer "F.Cu") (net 13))
 (segment (start 97.89 90.87) (end 97.89 91.7698) (width 0.127) (layer "F.Cu") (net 13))
 (segment (start 100.435 92.2818) (end 100.82 91.8968) (width 0.127) (layer "F.Cu") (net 17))
 (segment (start 100.82 90.49) (end 100.96 90.35) (width 0.127) (layer "F.Cu") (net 17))
 (segment (start 100.153 92.5636) (end 100.435 92.2818) (width 0.127) (layer "F.Cu") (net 17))
 (segment (start 100.82 91.8968) (end 100.82 90.49) (width 0.127) (layer "F.Cu") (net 17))
 (segment (start 99.45 92.65) (end 99.5364 92.5636) (width 0.127) (layer "F.Cu") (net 17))
 (segment (start 104.85 92.65) (end 103.9352 92.65) (width 0.127) (layer "F.Cu") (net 17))
 (segment (start 100.96 90.35) (end 101.58 90.35) (width 0.127) (layer "F.Cu") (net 17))
 (segment (start 99.5364 92.5636) (end 100.153 92.5636) (width 0.127) (layer "F.Cu") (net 17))
 (segment (start 103.9352 92.65) (end 103.906 92.6792) (width 0.127) (layer "F.Cu") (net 17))
 (via (at 99.45 92.65) (size 0.45) (drill 0.3) (layers "F.Cu" "B.Cu") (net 17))
 (via (at 104.85 92.65) (size 0.45) (drill 0.3) (layers "F.Cu" "B.Cu") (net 17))
 (segment (start 99.45 92.65) (end 99.57 92.53) (width 0.127) (layer "B.Cu") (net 17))
 (segment (start 104.85 92.65) (end 99.45 92.65) (width 0.127) (layer "B.Cu") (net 17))
 (segment (start 102.464 95.3037) (end 103.088 94.6792) (width 0.127) (layer "F.Cu") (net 31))
 (segment (start 101.215 95.0948) (end 101.142 95.0219) (width 0.25) (layer "F.Cu") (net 31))
 (segment (start 101.424 95.3037) (end 102.464 95.3037) (width 0.127) (layer "F.Cu") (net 31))
 (segment (start 103.088 94.6792) (end 103.906 94.6792) (width 0.127) (layer "F.Cu") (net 31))
 (segment (start 101.288 95.1677) (end 101.215 95.0948) (width 0.25) (layer "F.Cu") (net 31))
 (segment (start 101.288 95.1677) (end 101.424 95.3037) (width 0.127) (layer "F.Cu") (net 31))
 (segment (start 101.215 95.0948) (end 101.1421 95.0219) (width 0.25) (layer "F.Cu") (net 31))
 (segment (start 101.152 95.0317) (end 101.288 95.1677) (width 0.127) (layer "F.Cu") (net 31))
 (segment (start 101.496 94.6683) (end 101.785 94.9574) (width 0.127) (layer "F.Cu") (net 32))
 (segment (start 101.4956 94.6683) (end 101.496 94.6683) (width 0.25) (layer "F.Cu") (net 32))
 (segment (start 101.785 94.9574) (end 102.348 94.9574) (width 0.127) (layer "F.Cu") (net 32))
 (segment (start 103.126 94.1792) (end 103.906 94.1792) (width 0.127) (layer "F.Cu") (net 32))
 (segment (start 102.348 94.9574) (end 103.126 94.1792) (width 0.127) (layer "F.Cu") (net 32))
 (segment (start 101.077 97.153) (end 103.051 95.1792) (width 0.127) (layer "F.Cu") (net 27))
 (segment (start 99.0667 96.4785) (end 99.7412 97.153) (width 0.127) (layer "F.Cu") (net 27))
 (segment (start 103.051 95.1792) (end 103.906 95.1792) (width 0.127) (layer "F.Cu") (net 27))
 (segment (start 99.7412 97.153) (end 101.077 97.153) (width 0.127) (layer "F.Cu") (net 27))
 (segment (start 98.5338 96.2862) (end 98.7375 96.0825) (width 0.127) (layer "F.Cu") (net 26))
 (segment (start 103.301 95.6792) (end 101.5 97.48) (width 0.127) (layer "F.Cu") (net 26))
 (segment (start 98.33 97.25) (end 98.33 96.49) (width 0.127) (layer "F.Cu") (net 26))
 (segment (start 98.5338 96.2862) (end 98.5519 96.2862) (width 0.25) (layer "F.Cu") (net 26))
 (segment (start 103.906 95.6792) (end 103.301 95.6792) (width 0.127) (layer "F.Cu") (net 26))
 (segment (start 98.56 97.48) (end 98.33 97.25) (width 0.127) (layer "F.Cu") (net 26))
 (segment (start 98.5519 96.2862) (end 98.7556 96.0825) (width 0.25) (layer "F.Cu") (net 26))
 (segment (start 101.5 97.48) (end 98.56 97.48) (width 0.127) (layer "F.Cu") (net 26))
 (segment (start 98.33 96.49) (end 98.5338 96.2862) (width 0.127) (layer "F.Cu") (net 26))
 (segment (start 101.891606 93.653614) (end 101.891606 93.648394) (width 0.25) (layer "F.Cu") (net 15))
 (segment (start 101.891606 93.648394) (end 103.3608 92.1792) (width 0.127) (layer "F.Cu") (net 15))
 (segment (start 103.3608 92.1792) (end 103.906 92.1792) (width 0.127) (layer "F.Cu") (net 15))
 (segment (start 100.493 89.437) (end 100.88 89.05) (width 0.127) (layer "F.Cu") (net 10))
 (segment (start 100.081 91.9282) (end 100.0813 91.9282) (width 0.25) (layer "F.Cu") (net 10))
 (segment (start 100.081 91.9283) (end 100.287 91.7225) (width 0.127) (layer "F.Cu") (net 10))
 (segment (start 100.88 89.05) (end 104.015 89.05) (width 0.127) (layer "F.Cu") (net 10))
 (segment (start 100.081 91.9282) (end 100.081 91.9283) (width 0.25) (layer "F.Cu") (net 10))
 (segment (start 100.287 91.7225) (end 100.081 91.9281) (width 0.25) (layer "F.Cu") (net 10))
 (segment (start 100.081 91.9281) (end 100.081 91.9282) (width 0.25) (layer "F.Cu") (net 10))
 (segment (start 100.493 91.5167) (end 100.493 89.437) (width 0.127) (layer "F.Cu") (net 10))
 (segment (start 100.287 91.7225) (end 100.493 91.5167) (width 0.127) (layer "F.Cu") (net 10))
 (segment (start 100.0813 91.9282) (end 100.0814 91.9283) (width 0.25) (layer "F.Cu") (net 10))
 (segment (start 104.015 89.05) (end 105.22 89.05) (width 0.127) (layer "F.Cu") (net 10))
 (segment (start 105.22 89.05) (end 105.75 88.52) (width 0.127) (layer "F.Cu") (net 10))
 (segment (start 98.402 95.718) (end 99.06 95.06) (width 0.127) (layer "F.Cu") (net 25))
 (segment (start 98.402 95.729) (end 98.402 95.718) (width 0.25) (layer "F.Cu") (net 25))
 (segment (start 99.06 95.06) (end 99.06 94.56) (width 0.127) (layer "F.Cu") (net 25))
 (segment (start 88.5924 97.7576) (end 88.5924 99.8474) (width 0.127) (layer "F.Cu") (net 25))
 (segment (start 89.027 97.323) (end 88.5924 97.7576) (width 0.127) (layer "F.Cu") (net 25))
 (segment (start 94.69 97.323) (end 89.027 97.323) (width 0.127) (layer "F.Cu") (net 25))
 (via (at 94.69 97.323) (size 0.45) (drill 0.3) (layers "F.Cu" "B.Cu") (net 25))
 (via (at 99.06 94.56) (size 0.45) (drill 0.3) (layers "F.Cu" "B.Cu") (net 25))
 (segment (start 99.06 97.29) (end 99.06 94.56) (width 0.127) (layer "B.Cu") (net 25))
 (segment (start 94.69 97.323) (end 99.027 97.323) (width 0.127) (layer "B.Cu") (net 25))
 (segment (start 99.027 97.323) (end 99.06 97.29) (width 0.127) (layer "B.Cu") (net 25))
 (segment (start 99.8705 95.8718) (end 99.66 95.6611) (width 0.127) (layer "F.Cu") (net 7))
 (segment (start 99.8705 95.8718) (end 99.8707 95.8718) (width 0.25) (layer "F.Cu") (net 7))
 (segment (start 100.081 96.0825) (end 99.8705 95.8718) (width 0.127) (layer "F.Cu") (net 7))
 (segment (start 99.8707 95.8718) (end 100.081 96.0825) (width 0.25) (layer "F.Cu") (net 7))
 (segment (start 99.66 95.6611) (end 99.66 95.09) (width 0.127) (layer "F.Cu") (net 7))
 (segment (start 100.0814 96.0825) (end 100.081 96.0825) (width 0.25) (layer "F.Cu") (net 7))
 (via (at 99.66 95.09) (size 0.45) (drill 0.3) (layers "F.Cu" "B.Cu") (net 7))
 (segment (start 99.31 99.52) (end 99.66 99.17) (width 0.127) (layer "B.Cu") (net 7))
 (segment (start 99.66 99.17) (end 99.66 95.09) (width 0.127) (layer "B.Cu") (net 7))
 (segment (start 94.8662 99.52) (end 99.31 99.52) (width 0.127) (layer "B.Cu") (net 7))
 (segment (start 94.5388 99.8474) (end 94.8662 99.52) (width 0.127) (layer "B.Cu") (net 7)))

